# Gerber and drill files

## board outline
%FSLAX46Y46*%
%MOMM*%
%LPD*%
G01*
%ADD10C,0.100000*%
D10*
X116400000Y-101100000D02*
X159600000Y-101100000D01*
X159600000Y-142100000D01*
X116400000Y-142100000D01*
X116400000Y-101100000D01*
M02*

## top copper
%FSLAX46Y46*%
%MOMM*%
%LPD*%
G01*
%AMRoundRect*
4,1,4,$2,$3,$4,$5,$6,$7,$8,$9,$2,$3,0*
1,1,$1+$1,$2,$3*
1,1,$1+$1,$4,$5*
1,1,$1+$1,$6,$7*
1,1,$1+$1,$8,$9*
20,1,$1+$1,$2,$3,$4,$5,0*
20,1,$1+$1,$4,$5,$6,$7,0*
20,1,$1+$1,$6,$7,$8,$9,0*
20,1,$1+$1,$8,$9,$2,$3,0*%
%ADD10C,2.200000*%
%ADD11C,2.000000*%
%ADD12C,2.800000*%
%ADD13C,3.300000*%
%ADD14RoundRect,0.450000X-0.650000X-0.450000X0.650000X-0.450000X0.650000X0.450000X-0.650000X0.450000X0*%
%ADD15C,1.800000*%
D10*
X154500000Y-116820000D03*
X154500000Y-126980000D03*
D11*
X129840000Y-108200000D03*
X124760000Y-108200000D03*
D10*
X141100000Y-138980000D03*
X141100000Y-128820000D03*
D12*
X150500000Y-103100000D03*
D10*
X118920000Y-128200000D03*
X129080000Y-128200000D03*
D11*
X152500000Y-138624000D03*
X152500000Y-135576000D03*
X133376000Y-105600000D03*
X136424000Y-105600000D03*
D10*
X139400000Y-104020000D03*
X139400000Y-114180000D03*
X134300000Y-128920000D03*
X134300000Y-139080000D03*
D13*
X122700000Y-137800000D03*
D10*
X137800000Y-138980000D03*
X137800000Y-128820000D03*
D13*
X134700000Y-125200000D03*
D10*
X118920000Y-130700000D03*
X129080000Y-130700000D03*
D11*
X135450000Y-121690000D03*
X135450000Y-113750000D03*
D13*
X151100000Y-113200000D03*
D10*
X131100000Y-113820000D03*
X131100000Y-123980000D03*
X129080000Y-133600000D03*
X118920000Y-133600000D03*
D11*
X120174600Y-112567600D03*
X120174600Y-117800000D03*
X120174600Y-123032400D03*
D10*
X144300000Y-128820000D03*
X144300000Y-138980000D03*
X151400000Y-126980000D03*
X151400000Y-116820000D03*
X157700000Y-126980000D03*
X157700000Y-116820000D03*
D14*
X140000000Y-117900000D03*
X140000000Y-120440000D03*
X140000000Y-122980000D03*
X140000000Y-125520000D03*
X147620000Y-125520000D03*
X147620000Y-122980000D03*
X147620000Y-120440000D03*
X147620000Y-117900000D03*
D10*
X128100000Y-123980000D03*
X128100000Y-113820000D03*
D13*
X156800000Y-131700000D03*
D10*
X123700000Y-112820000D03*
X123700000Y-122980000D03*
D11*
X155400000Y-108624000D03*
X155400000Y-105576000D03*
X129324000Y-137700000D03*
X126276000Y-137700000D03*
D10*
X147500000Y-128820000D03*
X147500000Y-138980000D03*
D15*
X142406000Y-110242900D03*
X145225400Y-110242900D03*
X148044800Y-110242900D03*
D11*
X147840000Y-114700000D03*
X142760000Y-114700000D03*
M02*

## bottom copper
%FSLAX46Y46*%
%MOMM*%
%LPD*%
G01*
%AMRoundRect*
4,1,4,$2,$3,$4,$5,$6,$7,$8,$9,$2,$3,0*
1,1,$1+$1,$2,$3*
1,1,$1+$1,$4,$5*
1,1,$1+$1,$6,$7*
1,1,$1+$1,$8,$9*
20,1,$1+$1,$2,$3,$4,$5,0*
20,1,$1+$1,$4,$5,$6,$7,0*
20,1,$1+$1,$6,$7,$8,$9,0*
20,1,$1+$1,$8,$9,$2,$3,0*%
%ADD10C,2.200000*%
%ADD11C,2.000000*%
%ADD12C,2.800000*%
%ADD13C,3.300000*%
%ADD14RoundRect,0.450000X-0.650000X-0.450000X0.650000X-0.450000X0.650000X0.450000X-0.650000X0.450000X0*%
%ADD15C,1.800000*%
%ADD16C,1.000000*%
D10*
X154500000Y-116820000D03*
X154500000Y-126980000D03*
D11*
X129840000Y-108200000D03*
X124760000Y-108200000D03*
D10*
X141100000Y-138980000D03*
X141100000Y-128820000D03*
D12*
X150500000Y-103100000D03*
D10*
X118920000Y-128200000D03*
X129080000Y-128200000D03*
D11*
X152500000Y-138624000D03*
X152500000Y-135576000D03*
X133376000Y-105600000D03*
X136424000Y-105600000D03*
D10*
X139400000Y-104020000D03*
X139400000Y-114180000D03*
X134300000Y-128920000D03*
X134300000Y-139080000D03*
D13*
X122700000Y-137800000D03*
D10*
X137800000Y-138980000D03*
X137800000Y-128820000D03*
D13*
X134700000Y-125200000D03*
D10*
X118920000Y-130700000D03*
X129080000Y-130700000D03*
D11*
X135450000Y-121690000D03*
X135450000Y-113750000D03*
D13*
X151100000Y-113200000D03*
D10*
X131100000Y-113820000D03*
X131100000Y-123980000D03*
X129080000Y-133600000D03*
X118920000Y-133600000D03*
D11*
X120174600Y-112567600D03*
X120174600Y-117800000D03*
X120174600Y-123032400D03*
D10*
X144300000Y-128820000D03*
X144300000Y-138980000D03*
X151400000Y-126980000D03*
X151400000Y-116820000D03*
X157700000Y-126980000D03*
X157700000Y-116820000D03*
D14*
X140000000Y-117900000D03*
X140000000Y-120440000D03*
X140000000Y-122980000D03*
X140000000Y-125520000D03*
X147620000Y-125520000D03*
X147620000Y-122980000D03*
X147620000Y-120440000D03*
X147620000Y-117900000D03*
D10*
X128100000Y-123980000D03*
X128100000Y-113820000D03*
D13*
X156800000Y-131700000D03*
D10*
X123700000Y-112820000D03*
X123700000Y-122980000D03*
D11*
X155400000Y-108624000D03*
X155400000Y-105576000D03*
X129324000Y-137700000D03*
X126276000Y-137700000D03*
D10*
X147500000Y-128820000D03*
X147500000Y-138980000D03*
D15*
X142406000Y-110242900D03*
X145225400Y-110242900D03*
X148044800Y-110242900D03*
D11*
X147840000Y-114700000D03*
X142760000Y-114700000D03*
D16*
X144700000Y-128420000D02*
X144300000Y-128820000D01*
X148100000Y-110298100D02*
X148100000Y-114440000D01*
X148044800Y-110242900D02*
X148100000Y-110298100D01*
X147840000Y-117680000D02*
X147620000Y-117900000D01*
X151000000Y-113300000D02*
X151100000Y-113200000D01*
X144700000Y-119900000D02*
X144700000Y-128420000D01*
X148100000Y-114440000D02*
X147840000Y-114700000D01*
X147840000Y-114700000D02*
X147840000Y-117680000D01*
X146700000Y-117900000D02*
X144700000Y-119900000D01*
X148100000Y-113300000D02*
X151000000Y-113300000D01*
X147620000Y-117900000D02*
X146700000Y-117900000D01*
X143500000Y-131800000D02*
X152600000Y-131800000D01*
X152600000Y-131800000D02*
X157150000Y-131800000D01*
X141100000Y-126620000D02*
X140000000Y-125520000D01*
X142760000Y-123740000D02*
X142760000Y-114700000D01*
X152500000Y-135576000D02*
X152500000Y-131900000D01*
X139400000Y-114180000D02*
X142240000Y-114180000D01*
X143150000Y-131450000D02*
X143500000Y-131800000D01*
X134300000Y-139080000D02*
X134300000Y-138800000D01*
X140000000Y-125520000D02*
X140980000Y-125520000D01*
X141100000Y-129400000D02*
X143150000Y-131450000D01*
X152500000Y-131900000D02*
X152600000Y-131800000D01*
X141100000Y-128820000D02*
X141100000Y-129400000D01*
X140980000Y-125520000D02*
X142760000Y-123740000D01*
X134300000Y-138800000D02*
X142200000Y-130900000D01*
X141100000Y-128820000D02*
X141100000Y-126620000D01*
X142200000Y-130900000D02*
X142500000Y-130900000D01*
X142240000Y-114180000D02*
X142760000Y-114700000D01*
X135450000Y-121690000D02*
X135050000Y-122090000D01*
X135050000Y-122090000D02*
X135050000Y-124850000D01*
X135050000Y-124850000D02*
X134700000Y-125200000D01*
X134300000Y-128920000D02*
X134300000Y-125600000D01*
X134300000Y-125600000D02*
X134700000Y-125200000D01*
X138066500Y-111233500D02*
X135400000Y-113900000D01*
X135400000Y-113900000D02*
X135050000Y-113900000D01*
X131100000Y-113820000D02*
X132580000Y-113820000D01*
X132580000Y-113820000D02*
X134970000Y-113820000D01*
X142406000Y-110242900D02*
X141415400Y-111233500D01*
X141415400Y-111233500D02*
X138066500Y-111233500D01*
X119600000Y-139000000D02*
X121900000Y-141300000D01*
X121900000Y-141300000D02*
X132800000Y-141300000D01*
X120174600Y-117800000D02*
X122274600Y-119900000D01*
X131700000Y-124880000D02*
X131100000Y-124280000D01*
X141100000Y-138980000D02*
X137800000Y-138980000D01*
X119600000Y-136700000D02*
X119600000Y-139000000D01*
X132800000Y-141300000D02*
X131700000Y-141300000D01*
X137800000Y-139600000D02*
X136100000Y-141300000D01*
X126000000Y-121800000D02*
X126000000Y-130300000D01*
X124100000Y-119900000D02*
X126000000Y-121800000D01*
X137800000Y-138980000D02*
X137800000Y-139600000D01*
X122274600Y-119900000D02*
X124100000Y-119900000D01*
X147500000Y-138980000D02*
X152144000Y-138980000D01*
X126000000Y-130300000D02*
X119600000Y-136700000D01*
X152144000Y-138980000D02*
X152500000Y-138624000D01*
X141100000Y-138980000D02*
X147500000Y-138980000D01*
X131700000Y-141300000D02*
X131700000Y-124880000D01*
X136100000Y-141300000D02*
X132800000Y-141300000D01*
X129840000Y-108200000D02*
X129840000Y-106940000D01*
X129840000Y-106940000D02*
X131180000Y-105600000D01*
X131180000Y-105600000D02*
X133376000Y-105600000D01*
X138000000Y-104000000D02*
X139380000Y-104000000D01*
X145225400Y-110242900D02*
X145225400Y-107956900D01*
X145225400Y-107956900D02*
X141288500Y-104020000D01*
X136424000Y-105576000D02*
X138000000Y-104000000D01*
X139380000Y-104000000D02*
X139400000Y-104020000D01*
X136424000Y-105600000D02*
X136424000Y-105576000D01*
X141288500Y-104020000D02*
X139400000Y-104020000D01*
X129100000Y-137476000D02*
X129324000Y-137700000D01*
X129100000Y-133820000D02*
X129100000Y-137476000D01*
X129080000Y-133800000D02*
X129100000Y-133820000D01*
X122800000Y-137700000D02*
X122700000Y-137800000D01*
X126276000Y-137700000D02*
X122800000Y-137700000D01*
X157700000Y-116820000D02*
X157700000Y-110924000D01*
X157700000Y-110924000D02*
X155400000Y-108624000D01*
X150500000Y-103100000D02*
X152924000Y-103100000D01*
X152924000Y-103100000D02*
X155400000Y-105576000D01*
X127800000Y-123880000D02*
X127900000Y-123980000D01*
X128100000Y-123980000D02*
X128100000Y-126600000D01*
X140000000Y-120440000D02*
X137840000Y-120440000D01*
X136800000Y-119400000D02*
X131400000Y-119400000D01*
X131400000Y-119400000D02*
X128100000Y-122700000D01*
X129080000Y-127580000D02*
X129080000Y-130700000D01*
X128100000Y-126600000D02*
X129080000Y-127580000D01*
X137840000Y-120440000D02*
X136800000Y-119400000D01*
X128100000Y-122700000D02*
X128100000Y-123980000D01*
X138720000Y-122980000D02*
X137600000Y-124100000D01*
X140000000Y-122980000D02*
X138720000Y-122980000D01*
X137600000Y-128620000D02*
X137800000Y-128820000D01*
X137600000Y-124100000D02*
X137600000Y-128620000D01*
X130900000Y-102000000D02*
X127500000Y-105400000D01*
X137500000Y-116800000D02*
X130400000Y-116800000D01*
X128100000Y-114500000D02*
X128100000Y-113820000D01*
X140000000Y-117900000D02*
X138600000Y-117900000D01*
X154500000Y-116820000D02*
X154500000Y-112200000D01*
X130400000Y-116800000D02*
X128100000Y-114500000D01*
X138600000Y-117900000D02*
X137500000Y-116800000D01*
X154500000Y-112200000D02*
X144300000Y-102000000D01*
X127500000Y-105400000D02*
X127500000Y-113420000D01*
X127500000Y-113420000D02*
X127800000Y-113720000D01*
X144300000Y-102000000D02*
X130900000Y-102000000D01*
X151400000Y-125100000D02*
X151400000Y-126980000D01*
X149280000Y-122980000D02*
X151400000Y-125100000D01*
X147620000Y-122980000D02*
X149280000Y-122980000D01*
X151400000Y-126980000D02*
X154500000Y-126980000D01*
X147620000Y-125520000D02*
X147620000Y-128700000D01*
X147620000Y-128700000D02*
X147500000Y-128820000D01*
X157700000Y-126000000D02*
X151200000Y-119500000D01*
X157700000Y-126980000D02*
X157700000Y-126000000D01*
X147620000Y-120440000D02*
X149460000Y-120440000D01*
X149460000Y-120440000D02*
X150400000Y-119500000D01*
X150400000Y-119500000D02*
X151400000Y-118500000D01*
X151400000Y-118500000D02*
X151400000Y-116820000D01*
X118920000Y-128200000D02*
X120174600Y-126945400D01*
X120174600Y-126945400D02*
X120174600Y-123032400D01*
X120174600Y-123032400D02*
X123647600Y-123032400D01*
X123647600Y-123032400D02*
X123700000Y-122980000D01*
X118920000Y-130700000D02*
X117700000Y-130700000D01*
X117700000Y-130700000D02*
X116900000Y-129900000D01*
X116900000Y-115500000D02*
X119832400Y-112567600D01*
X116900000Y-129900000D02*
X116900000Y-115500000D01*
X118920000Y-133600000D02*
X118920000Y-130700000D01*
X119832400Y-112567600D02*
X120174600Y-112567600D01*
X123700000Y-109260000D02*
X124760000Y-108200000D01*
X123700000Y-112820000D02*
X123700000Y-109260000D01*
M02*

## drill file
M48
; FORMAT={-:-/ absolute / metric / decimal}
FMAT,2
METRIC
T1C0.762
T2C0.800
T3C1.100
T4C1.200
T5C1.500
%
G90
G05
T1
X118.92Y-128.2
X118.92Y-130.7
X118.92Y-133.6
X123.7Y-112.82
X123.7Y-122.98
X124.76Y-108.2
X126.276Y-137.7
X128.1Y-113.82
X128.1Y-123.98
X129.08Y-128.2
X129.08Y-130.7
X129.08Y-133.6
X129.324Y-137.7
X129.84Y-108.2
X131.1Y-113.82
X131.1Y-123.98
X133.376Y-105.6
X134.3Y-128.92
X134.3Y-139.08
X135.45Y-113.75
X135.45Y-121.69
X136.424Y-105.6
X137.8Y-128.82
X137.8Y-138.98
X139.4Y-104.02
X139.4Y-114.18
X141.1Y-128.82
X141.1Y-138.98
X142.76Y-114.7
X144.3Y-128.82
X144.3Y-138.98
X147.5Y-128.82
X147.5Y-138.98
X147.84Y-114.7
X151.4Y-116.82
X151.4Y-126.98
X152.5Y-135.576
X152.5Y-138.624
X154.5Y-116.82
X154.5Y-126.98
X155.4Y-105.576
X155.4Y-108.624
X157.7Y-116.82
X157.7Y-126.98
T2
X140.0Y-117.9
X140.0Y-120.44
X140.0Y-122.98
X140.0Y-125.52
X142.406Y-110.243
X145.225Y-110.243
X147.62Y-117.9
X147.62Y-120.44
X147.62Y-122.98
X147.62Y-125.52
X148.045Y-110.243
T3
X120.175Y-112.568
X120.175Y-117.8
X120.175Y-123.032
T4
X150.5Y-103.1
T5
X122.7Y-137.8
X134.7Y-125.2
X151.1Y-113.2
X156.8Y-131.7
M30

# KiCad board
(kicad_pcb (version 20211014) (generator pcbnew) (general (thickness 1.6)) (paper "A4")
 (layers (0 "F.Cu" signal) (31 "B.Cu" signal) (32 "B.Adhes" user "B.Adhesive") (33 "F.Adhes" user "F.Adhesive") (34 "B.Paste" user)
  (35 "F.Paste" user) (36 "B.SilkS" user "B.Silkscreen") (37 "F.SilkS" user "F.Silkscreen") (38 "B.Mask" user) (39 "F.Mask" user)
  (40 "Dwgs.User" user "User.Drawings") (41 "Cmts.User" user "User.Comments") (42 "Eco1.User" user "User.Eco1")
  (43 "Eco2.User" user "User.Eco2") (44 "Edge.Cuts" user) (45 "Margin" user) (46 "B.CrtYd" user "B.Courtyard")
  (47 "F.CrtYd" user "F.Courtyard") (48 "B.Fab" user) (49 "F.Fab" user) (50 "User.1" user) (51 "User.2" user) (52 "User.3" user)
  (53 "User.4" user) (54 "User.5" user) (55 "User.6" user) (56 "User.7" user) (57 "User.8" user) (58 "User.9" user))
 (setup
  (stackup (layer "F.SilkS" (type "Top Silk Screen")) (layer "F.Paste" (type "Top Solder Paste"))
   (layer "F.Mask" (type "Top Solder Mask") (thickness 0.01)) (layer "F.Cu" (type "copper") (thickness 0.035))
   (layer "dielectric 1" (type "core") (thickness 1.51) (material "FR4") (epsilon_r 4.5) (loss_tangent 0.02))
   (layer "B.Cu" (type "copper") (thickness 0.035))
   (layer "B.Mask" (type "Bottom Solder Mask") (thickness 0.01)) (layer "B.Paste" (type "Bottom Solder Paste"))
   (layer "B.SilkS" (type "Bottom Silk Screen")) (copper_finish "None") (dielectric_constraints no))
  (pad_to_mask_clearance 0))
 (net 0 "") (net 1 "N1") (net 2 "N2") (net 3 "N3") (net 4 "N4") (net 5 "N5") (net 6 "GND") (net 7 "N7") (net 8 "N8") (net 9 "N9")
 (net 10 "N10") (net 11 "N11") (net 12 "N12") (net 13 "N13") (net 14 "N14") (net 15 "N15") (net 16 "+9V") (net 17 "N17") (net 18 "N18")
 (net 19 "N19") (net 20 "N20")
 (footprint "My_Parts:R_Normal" (layer "F.Cu") (at 154.5 121.9 -90)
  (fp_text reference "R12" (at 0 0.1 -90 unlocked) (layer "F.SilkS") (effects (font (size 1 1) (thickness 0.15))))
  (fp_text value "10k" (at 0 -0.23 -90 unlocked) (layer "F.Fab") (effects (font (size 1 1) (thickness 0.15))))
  (pad "1" thru_hole circle (at -5.08 0 270) (size 2.2 2.2) (drill 0.762) (layers *.Cu *.Mask) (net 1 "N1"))
  (pad "2" thru_hole circle (at 5.08 0 270) (size 2.2 2.2) (drill 0.762) (layers *.Cu *.Mask) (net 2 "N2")))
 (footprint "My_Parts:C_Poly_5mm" (layer "F.Cu") (at 127.3 108.2 180)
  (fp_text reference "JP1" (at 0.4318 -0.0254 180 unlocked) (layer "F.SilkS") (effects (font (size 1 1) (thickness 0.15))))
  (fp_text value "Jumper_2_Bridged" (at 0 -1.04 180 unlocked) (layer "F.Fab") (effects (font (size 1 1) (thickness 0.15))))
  (pad "1" thru_hole circle (at -2.54 0 180) (size 2 2) (drill 0.762) (layers *.Cu *.Mask) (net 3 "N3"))
  (pad "2" thru_hole circle (at 2.54 0 180) (size 2 2) (drill 0.762) (layers *.Cu *.Mask) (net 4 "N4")))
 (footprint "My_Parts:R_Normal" (layer "F.Cu") (at 141.1 133.9 90)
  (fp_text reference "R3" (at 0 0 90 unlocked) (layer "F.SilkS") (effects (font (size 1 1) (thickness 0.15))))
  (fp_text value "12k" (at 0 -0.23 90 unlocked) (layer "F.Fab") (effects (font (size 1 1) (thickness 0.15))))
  (pad "1" thru_hole circle (at -5.08 0 90) (size 2.2 2.2) (drill 0.762) (layers *.Cu *.Mask) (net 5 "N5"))
  (pad "2" thru_hole circle (at 5.08 0 90) (size 2.2 2.2) (drill 0.762) (layers *.Cu *.Mask) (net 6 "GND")))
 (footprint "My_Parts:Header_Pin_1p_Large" (layer "F.Cu") (at 150.5 103.1)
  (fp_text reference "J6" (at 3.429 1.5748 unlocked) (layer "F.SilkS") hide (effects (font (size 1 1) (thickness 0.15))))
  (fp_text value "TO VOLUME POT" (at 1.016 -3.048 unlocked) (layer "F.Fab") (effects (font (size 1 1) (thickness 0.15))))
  (pad "1" thru_hole circle (at 0 0) (size 2.8 2.8) (drill 1.2) (layers *.Cu *.Mask) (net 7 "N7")))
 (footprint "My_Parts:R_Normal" (layer "F.Cu") (at 124 128.2)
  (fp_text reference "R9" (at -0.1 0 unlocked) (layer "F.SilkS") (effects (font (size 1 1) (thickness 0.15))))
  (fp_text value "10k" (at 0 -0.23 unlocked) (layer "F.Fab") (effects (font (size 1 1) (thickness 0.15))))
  (pad "1" thru_hole circle (at -5.08 0) (size 2.2 2.2) (drill 0.762) (layers *.Cu *.Mask) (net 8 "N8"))
  (pad "2" thru_hole circle (at 5.08 0) (size 2.2 2.2) (drill 0.762) (layers *.Cu *.Mask) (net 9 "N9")))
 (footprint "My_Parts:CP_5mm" (layer "F.Cu") (at 152.5 137.1 90)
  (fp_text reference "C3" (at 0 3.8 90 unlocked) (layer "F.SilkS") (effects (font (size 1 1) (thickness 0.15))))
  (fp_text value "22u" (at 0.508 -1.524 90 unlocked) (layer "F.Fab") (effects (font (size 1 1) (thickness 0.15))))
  (pad "1" thru_hole circle (at -1.524 0 90) (size 2 2) (drill 0.762) (layers *.Cu *.Mask) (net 5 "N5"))
  (pad "2" thru_hole circle (at 1.524 0 90) (size 2 2) (drill 0.762) (layers *.Cu *.Mask) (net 6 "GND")))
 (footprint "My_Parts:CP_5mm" (layer "F.Cu") (at 134.9 105.6)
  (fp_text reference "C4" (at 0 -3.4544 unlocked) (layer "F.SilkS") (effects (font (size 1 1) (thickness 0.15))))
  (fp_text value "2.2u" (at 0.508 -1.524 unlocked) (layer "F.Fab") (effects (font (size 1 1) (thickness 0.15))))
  (pad "1" thru_hole circle (at -1.524 0) (size 2 2) (drill 0.762) (layers *.Cu *.Mask) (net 3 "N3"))
  (pad "2" thru_hole circle (at 1.524 0) (size 2 2) (drill 0.762) (layers *.Cu *.Mask) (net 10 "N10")))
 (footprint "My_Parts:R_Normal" (layer "F.Cu") (at 139.4 109.1 -90)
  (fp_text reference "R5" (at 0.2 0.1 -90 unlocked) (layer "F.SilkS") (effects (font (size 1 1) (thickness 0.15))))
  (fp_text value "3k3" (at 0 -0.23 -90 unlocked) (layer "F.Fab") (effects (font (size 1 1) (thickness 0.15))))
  (pad "1" thru_hole circle (at -5.08 0 270) (size 2.2 2.2) (drill 0.762) (layers *.Cu *.Mask) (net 10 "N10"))
  (pad "2" thru_hole circle (at 5.08 0 270) (size 2.2 2.2) (drill 0.762) (layers *.Cu *.Mask) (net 6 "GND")))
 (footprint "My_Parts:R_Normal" (layer "F.Cu") (at 134.3 134 -90)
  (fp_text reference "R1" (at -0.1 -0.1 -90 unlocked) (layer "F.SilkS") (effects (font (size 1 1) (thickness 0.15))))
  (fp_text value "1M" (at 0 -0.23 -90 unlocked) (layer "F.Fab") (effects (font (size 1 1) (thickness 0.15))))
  (pad "1" thru_hole circle (at -5.08 0 270) (size 2.2 2.2) (drill 0.762) (layers *.Cu *.Mask) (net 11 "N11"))
  (pad "2" thru_hole circle (at 5.08 0 270) (size 2.2 2.2) (drill 0.762) (layers *.Cu *.Mask) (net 6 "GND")))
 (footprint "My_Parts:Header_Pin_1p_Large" (layer "F.Cu") (at 122.7 137.8)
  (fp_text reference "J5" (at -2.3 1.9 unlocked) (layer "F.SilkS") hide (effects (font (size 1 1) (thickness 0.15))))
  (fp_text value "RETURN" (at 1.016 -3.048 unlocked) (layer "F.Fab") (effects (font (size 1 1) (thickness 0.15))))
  (pad "1" thru_hole circle (at 0 0) (size 3.3 3.3) (drill 1.5) (layers *.Cu *.Mask) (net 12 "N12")))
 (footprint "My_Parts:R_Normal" (layer "F.Cu") (at 137.8 133.9 90)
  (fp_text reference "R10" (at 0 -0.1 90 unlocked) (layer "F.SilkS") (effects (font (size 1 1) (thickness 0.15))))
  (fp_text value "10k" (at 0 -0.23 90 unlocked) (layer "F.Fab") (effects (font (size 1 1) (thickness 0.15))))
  (pad "1" thru_hole circle (at -5.08 0 90) (size 2.2 2.2) (drill 0.762) (layers *.Cu *.Mask) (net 5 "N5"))
  (pad "2" thru_hole circle (at 5.08 0 90) (size 2.2 2.2) (drill 0.762) (layers *.Cu *.Mask) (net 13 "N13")))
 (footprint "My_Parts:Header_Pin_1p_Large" (layer "F.Cu") (at 134.7 125.2)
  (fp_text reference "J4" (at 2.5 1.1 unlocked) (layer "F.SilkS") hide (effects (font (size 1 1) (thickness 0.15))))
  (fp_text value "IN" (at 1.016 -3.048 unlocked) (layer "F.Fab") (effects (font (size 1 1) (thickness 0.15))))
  (pad "1" thru_hole circle (at 0 0) (size 3.3 3.3) (drill 1.5) (layers *.Cu *.Mask) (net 11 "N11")))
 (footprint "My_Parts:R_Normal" (layer "F.Cu") (at 124 130.7)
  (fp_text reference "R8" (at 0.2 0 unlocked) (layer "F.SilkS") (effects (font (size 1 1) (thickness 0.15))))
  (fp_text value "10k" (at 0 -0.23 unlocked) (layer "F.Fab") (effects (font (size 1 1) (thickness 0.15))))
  (pad "1" thru_hole circle (at -5.08 0) (size 2.2 2.2) (drill 0.762) (layers *.Cu *.Mask) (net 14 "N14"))
  (pad "2" thru_hole circle (at 5.08 0) (size 2.2 2.2) (drill 0.762) (layers *.Cu *.Mask) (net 9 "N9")))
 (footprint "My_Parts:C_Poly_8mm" (layer "F.Cu") (at 135.45 119.15 90)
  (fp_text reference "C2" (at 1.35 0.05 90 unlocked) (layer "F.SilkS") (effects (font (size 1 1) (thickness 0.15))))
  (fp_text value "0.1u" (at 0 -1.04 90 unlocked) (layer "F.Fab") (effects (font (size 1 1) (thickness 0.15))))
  (pad "1" thru_hole circle (at -2.54 0 90) (size 2 2) (drill 0.762) (layers *.Cu *.Mask) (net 11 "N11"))
  (pad "2" thru_hole circle (at 5.4 0 90) (size 2 2) (drill 0.762) (layers *.Cu *.Mask) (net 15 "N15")))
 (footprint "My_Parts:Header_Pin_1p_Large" (layer "F.Cu") (at 151.1 113.2)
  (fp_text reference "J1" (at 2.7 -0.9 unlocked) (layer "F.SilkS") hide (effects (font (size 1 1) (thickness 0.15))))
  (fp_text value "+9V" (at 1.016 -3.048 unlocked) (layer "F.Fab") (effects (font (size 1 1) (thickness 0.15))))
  (pad "1" thru_hole circle (at 0 0) (size 3.3 3.3) (drill 1.5) (layers *.Cu *.Mask) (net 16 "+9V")))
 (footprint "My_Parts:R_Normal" (layer "F.Cu") (at 131.1 118.9 -90)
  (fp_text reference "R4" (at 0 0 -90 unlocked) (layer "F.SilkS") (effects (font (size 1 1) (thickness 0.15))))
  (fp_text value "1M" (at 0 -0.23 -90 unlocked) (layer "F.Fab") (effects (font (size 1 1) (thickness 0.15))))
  (pad "1" thru_hole circle (at -5.08 0 270) (size 2.2 2.2) (drill 0.762) (layers *.Cu *.Mask) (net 15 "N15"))
  (pad "2" thru_hole circle (at 5.08 0 270) (size 2.2 2.2) (drill 0.762) (layers *.Cu *.Mask) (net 5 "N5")))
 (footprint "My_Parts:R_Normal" (layer "F.Cu") (at 124 133.6 180)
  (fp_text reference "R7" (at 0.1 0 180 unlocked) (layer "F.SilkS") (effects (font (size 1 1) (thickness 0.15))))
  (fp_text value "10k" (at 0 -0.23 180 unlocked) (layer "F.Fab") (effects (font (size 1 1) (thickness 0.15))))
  (pad "1" thru_hole circle (at -5.08 0 180) (size 2.2 2.2) (drill 0.762) (layers *.Cu *.Mask) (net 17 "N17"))
  (pad "2" thru_hole circle (at 5.08 0 180) (size 2.2 2.2) (drill 0.762) (layers *.Cu *.Mask) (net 14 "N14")))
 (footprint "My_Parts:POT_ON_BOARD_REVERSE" (layer "F.Cu") (at 120.2 117.8 90)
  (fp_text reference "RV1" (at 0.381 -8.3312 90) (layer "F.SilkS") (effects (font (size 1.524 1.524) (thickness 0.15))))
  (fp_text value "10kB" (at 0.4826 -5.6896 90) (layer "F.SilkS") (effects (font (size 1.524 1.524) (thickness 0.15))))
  (pad "1" thru_hole circle (at 5.2324 -0.0254 90) (size 2 2) (drill 1.09982) (layers *.Cu "F.Paste" "F.Mask") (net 14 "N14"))
  (pad "2" thru_hole circle (at 0 -0.0254 90) (size 2 2) (drill 1.09982) (layers *.Cu "F.Paste" "F.Mask") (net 5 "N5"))
  (pad "3" thru_hole circle (at -5.2324 -0.0254 90) (size 2 2) (drill 1.09982) (layers *.Cu "F.Paste" "F.Mask") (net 8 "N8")))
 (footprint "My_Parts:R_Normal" (layer "F.Cu") (at 144.3 133.9 -90)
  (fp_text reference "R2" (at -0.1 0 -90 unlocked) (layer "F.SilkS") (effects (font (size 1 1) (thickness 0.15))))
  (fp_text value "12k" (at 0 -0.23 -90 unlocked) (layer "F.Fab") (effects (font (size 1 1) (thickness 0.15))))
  (pad "1" thru_hole circle (at -5.08 0 270) (size 2.2 2.2) (drill 0.762) (layers *.Cu *.Mask) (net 16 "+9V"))
  (pad "2" thru_hole circle (at 5.08 0 270) (size 2.2 2.2) (drill 0.762) (layers *.Cu *.Mask) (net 5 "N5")))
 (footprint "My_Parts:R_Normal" (layer "F.Cu") (at 151.4 121.9 90)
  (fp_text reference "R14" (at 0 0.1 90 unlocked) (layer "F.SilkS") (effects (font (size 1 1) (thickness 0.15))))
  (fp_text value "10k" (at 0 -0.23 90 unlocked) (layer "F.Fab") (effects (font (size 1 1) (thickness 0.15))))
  (pad "1" thru_hole circle (at -5.08 0 90) (size 2.2 2.2) (drill 0.762) (layers *.Cu *.Mask) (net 2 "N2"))
  (pad "2" thru_hole circle (at 5.08 0 90) (size 2.2 2.2) (drill 0.762) (layers *.Cu *.Mask) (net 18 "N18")))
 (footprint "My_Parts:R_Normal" (layer "F.Cu") (at 157.7 121.9 90)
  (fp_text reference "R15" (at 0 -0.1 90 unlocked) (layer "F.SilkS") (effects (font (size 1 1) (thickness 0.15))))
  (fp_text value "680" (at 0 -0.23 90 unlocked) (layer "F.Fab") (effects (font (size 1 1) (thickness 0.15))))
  (pad "1" thru_hole circle (at -5.08 0 90) (size 2.2 2.2) (drill 0.762) (layers *.Cu *.Mask) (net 18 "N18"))
  (pad "2" thru_hole circle (at 5.08 0 90) (size 2.2 2.2) (drill 0.762) (layers *.Cu *.Mask) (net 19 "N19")))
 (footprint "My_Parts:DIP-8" (layer "F.Cu") (at 141.27 118.4)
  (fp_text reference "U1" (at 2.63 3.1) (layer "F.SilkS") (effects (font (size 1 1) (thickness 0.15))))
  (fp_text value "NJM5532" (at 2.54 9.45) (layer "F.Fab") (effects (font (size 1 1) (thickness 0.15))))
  (pad "1" thru_hole roundrect (at -1.27 -0.5) (size 2.2 1.8) (drill 0.8) (layers *.Cu *.Mask) (roundrect_rratio 0.25) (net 1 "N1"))
  (pad "2" thru_hole roundrect (at -1.27 2.04) (size 2.2 1.8) (drill 0.8) (layers *.Cu *.Mask) (roundrect_rratio 0.25) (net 9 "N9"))
  (pad "3" thru_hole roundrect (at -1.27 4.58) (size 2.2 1.8) (drill 0.8) (layers *.Cu *.Mask) (roundrect_rratio 0.25) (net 13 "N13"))
  (pad "4" thru_hole roundrect (at -1.27 7.12) (size 2.2 1.8) (drill 0.8) (layers *.Cu *.Mask) (roundrect_rratio 0.25) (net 6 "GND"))
  (pad "5" thru_hole roundrect (at 6.35 7.12) (size 2.2 1.8) (drill 0.8) (layers *.Cu *.Mask) (roundrect_rratio 0.25) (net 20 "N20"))
  (pad "6" thru_hole roundrect (at 6.35 4.58) (size 2.2 1.8) (drill 0.8) (layers *.Cu *.Mask) (roundrect_rratio 0.25) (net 2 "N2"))
  (pad "7" thru_hole roundrect (at 6.35 2.04) (size 2.2 1.8) (drill 0.8) (layers *.Cu *.Mask) (roundrect_rratio 0.25) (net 18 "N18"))
  (pad "8" thru_hole roundrect (at 6.35 -0.5) (size 2.2 1.8) (drill 0.8) (layers *.Cu *.Mask) (roundrect_rratio 0.25) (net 16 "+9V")))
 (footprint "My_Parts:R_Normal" (layer "F.Cu") (at 128.1 118.9 90)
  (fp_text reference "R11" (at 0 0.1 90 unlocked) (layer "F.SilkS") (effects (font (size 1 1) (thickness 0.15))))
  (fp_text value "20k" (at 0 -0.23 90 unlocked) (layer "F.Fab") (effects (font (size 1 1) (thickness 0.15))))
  (pad "1" thru_hole circle (at -5.08 0 90) (size 2.2 2.2) (drill 0.762) (layers *.Cu *.Mask) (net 9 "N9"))
  (pad "2" thru_hole circle (at 5.08 0 90) (size 2.2 2.2) (drill 0.762) (layers *.Cu *.Mask) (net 1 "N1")))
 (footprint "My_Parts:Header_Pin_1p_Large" (layer "F.Cu") (at 156.8 131.7)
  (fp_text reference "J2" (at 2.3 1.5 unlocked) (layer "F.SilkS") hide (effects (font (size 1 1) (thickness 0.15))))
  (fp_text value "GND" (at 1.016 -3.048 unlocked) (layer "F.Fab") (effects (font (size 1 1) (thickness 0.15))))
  (pad "1" thru_hole circle (at 0 0) (size 3.3 3.3) (drill 1.5) (layers *.Cu *.Mask) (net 6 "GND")))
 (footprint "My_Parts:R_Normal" (layer "F.Cu") (at 123.7 117.9 -90)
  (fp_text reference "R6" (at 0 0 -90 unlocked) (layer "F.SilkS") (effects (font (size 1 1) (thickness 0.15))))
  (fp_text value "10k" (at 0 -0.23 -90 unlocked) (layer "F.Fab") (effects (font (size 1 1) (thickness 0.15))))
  (pad "1" thru_hole circle (at -5.08 0 270) (size 2.2 2.2) (drill 0.762) (layers *.Cu *.Mask) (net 4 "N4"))
  (pad "2" thru_hole circle (at 5.08 0 270) (size 2.2 2.2) (drill 0.762) (layers *.Cu *.Mask) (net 8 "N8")))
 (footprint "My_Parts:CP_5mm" (layer "F.Cu") (at 155.4 107.1 90)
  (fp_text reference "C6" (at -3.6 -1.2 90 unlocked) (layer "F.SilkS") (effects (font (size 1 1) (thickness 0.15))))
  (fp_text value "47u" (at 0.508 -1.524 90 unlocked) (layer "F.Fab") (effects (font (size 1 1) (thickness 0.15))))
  (pad "1" thru_hole circle (at -1.524 0 90) (size 2 2) (drill 0.762) (layers *.Cu *.Mask) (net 19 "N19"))
  (pad "2" thru_hole circle (at 1.524 0 90) (size 2 2) (drill 0.762) (layers *.Cu *.Mask) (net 7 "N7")))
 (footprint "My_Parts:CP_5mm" (layer "F.Cu") (at 127.8 137.7 180)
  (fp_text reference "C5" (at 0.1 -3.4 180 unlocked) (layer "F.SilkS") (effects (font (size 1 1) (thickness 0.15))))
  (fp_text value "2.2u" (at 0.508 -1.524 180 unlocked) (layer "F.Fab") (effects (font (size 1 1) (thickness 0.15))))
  (pad "1" thru_hole circle (at -1.524 0 180) (size 2 2) (drill 0.762) (layers *.Cu *.Mask) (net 17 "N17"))
  (pad "2" thru_hole circle (at 1.524 0 180) (size 2 2) (drill 0.762) (layers *.Cu *.Mask) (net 12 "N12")))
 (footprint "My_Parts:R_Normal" (layer "F.Cu") (at 147.5 133.9 -90)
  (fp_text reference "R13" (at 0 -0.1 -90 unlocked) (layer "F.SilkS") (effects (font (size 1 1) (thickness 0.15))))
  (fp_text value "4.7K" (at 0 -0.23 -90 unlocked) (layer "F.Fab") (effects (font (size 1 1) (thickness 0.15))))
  (pad "1" thru_hole circle (at -5.08 0 270) (size 2.2 2.2) (drill 0.762) (layers *.Cu *.Mask) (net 20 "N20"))
  (pad "2" thru_hole circle (at 5.08 0 270) (size 2.2 2.2) (drill 0.762) (layers *.Cu *.Mask) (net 5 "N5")))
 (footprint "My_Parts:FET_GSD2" (layer "F.Cu") (at 142.66 110.2175)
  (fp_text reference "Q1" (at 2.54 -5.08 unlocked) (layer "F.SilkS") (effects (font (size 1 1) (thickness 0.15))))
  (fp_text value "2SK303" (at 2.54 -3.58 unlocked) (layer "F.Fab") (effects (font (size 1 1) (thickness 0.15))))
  (pad "1" thru_hole circle (at -0.254 0.0254) (size 1.8 1.8) (drill 0.8) (layers *.Cu *.Mask) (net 15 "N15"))
  (pad "2" thru_hole circle (at 2.5654 0.0254) (size 1.8 1.8) (drill 0.8) (layers *.Cu *.Mask) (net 10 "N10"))
  (pad "3" thru_hole circle (at 5.3848 0.0254) (size 1.8 1.8) (drill 0.8) (layers *.Cu *.Mask) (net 16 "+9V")))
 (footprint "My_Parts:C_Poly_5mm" (layer "F.Cu") (at 145.3 114.7 180)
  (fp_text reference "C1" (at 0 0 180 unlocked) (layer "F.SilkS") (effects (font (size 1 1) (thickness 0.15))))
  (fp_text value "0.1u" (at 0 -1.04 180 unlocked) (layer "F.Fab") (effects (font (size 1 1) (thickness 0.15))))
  (pad "1" thru_hole circle (at -2.54 0 180) (size 2 2) (drill 0.762) (layers *.Cu *.Mask) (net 16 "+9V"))
  (pad "2" thru_hole circle (at 2.54 0 180) (size 2 2) (drill 0.762) (layers *.Cu *.Mask) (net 6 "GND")))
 (gr_rect (start 116.4 101.1) (end 159.6 142.1) (layer "Edge.Cuts") (width 0.1) (fill none))
 (segment (start 144.7 128.42) (end 144.3 128.82) (width 1) (layer "B.Cu") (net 16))
 (segment (start 148.1 110.2981) (end 148.1 114.44) (width 1) (layer "B.Cu") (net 16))
 (segment (start 148.0448 110.2429) (end 148.1 110.2981) (width 1) (layer "B.Cu") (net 16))
 (segment (start 147.84 117.68) (end 147.62 117.9) (width 1) (layer "B.Cu") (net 16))
 (segment (start 151 113.3) (end 151.1 113.2) (width 1) (layer "B.Cu") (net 16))
 (segment (start 144.7 119.9) (end 144.7 128.42) (width 1) (layer "B.Cu") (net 16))
 (segment (start 148.1 114.44) (end 147.84 114.7) (width 1) (layer "B.Cu") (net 16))
 (segment (start 147.84 114.7) (end 147.84 117.68) (width 1) (layer "B.Cu") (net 16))
 (segment (start 146.7 117.9) (end 144.7 119.9) (width 1) (layer "B.Cu") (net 16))
 (segment (start 148.1 113.3) (end 151 113.3) (width 1) (layer "B.Cu") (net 16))
 (segment (start 147.62 117.9) (end 146.7 117.9) (width 1) (layer "B.Cu") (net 16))
 (segment (start 143.5 131.8) (end 152.6 131.8) (width 1) (layer "B.Cu") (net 6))
 (segment (start 152.6 131.8) (end 157.15 131.8) (width 1) (layer "B.Cu") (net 6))
 (segment (start 141.1 126.62) (end 140 125.52) (width 1) (layer "B.Cu") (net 6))
 (segment (start 142.76 123.74) (end 142.76 114.7) (width 1) (layer "B.Cu") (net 6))
 (segment (start 152.5 135.576) (end 152.5 131.9) (width 1) (layer "B.Cu") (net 6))
 (segment (start 139.4 114.18) (end 142.24 114.18) (width 1) (layer "B.Cu") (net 6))
 (segment (start 143.15 131.45) (end 143.5 131.8) (width 1) (layer "B.Cu") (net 6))
 (segment (start 134.3 139.08) (end 134.3 138.8) (width 1) (layer "B.Cu") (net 6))
 (segment (start 140 125.52) (end 140.98 125.52) (width 1) (layer "B.Cu") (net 6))
 (segment (start 141.1 129.4) (end 143.15 131.45) (width 1) (layer "B.Cu") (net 6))
 (segment (start 152.5 131.9) (end 152.6 131.8) (width 1) (layer "B.Cu") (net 6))
 (segment (start 141.1 128.82) (end 141.1 129.4) (width 1) (layer "B.Cu") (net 6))
 (segment (start 140.98 125.52) (end 142.76 123.74) (width 1) (layer "B.Cu") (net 6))
 (segment (start 134.3 138.8) (end 142.2 130.9) (width 1) (layer "B.Cu") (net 6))
 (segment (start 141.1 128.82) (end 141.1 126.62) (width 1) (layer "B.Cu") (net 6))
 (segment (start 142.2 130.9) (end 142.5 130.9) (width 1) (layer "B.Cu") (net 6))
 (segment (start 142.24 114.18) (end 142.76 114.7) (width 1) (layer "B.Cu") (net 6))
 (segment (start 135.45 121.69) (end 135.05 122.09) (width 1) (layer "B.Cu") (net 11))
 (segment (start 135.05 122.09) (end 135.05 124.85) (width 1) (layer "B.Cu") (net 11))
 (segment (start 135.05 124.85) (end 134.7 125.2) (width 1) (layer "B.Cu") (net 11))
 (segment (start 134.3 128.92) (end 134.3 125.6) (width 1) (layer "B.Cu") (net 11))
 (segment (start 134.3 125.6) (end 134.7 125.2) (width 1) (layer "B.Cu") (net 11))
 (segment (start 138.0665 111.2335) (end 135.4 113.9) (width 1) (layer "B.Cu") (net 15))
 (segment (start 135.4 113.9) (end 135.05 113.9) (width 1) (layer "B.Cu") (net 15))
 (segment (start 131.1 113.82) (end 132.58 113.82) (width 1) (layer "B.Cu") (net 15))
 (segment (start 132.58 113.82) (end 134.97 113.82) (width 1) (layer "B.Cu") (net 15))
 (segment (start 142.406 110.2429) (end 141.4154 111.2335) (width 1) (layer "B.Cu") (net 15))
 (segment (start 141.4154 111.2335) (end 138.0665 111.2335) (width 1) (layer "B.Cu") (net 15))
 (segment (start 119.6 139) (end 121.9 141.3) (width 1) (layer "B.Cu") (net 5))
 (segment (start 121.9 141.3) (end 132.8 141.3) (width 1) (layer "B.Cu") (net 5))
 (segment (start 120.1746 117.8) (end 122.2746 119.9) (width 1) (layer "B.Cu") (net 5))
 (segment (start 131.7 124.88) (end 131.1 124.28) (width 1) (layer "B.Cu") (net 5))
 (segment (start 141.1 138.98) (end 137.8 138.98) (width 1) (layer "B.Cu") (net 5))
 (segment (start 119.6 136.7) (end 119.6 139) (width 1) (layer "B.Cu") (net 5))
 (segment (start 132.8 141.3) (end 131.7 141.3) (width 1) (layer "B.Cu") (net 5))
 (segment (start 137.8 139.6) (end 136.1 141.3) (width 1) (layer "B.Cu") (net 5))
 (segment (start 126 121.8) (end 126 130.3) (width 1) (layer "B.Cu") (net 5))
 (segment (start 124.1 119.9) (end 126 121.8) (width 1) (layer "B.Cu") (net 5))
 (segment (start 137.8 138.98) (end 137.8 139.6) (width 1) (layer "B.Cu") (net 5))
 (segment (start 122.2746 119.9) (end 124.1 119.9) (width 1) (layer "B.Cu") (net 5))
 (segment (start 147.5 138.98) (end 152.144 138.98) (width 1) (layer "B.Cu") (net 5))
 (segment (start 126 130.3) (end 119.6 136.7) (width 1) (layer "B.Cu") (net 5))
 (segment (start 152.144 138.98) (end 152.5 138.624) (width 1) (layer "B.Cu") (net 5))
 (segment (start 141.1 138.98) (end 147.5 138.98) (width 1) (layer "B.Cu") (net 5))
 (segment (start 131.7 141.3) (end 131.7 124.88) (width 1) (layer "B.Cu") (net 5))
 (segment (start 136.1 141.3) (end 132.8 141.3) (width 1) (layer "B.Cu") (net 5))
 (segment (start 129.84 108.2) (end 129.84 106.94) (width 1) (layer "B.Cu") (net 3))
 (segment (start 129.84 106.94) (end 131.18 105.6) (width 1) (layer "B.Cu") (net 3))
 (segment (start 131.18 105.6) (end 133.376 105.6) (width 1) (layer "B.Cu") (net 3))
 (segment (start 138 104) (end 139.38 104) (width 1) (layer "B.Cu") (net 10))
 (segment (start 145.2254 110.2429) (end 145.2254 107.9569) (width 1) (layer "B.Cu") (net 10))
 (segment (start 145.2254 107.9569) (end 141.2885 104.02) (width 1) (layer "B.Cu") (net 10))
 (segment (start 136.424 105.576) (end 138 104) (width 1) (layer "B.Cu") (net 10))
 (segment (start 139.38 104) (end 139.4 104.02) (width 1) (layer "B.Cu") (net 10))
 (segment (start 136.424 105.6) (end 136.424 105.576) (width 1) (layer "B.Cu") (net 10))
 (segment (start 141.2885 104.02) (end 139.4 104.02) (width 1) (layer "B.Cu") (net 10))
 (segment (start 129.1 137.476) (end 129.324 137.7) (width 1) (layer "B.Cu") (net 17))
 (segment (start 129.1 133.82) (end 129.1 137.476) (width 1) (layer "B.Cu") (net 17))
 (segment (start 129.08 133.8) (end 129.1 133.82) (width 1) (layer "B.Cu") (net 17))
 (segment (start 122.8 137.7) (end 122.7 137.8) (width 1) (layer "B.Cu") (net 12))
 (segment (start 126.276 137.7) (end 122.8 137.7) (width 1) (layer "B.Cu") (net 12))
 (segment (start 157.7 116.82) (end 157.7 110.924) (width 1) (layer "B.Cu") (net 19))
 (segment (start 157.7 110.924) (end 155.4 108.624) (width 1) (layer "B.Cu") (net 19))
 (segment (start 150.5 103.1) (end 152.924 103.1) (width 1) (layer "B.Cu") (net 7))
 (segment (start 152.924 103.1) (end 155.4 105.576) (width 1) (layer "B.Cu") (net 7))
 (segment (start 127.8 123.88) (end 127.9 123.98) (width 1) (layer "B.Cu") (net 9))
 (segment (start 128.1 123.98) (end 128.1 126.6) (width 1) (layer "B.Cu") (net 9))
 (segment (start 140 120.44) (end 137.84 120.44) (width 1) (layer "B.Cu") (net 9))
 (segment (start 136.8 119.4) (end 131.4 119.4) (width 1) (layer "B.Cu") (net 9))
 (segment (start 131.4 119.4) (end 128.1 122.7) (width 1) (layer "B.Cu") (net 9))
 (segment (start 129.08 127.58) (end 129.08 130.7) (width 1) (layer "B.Cu") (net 9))
 (segment (start 128.1 126.6) (end 129.08 127.58) (width 1) (layer "B.Cu") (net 9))
 (segment (start 137.84 120.44) (end 136.8 119.4) (width 1) (layer "B.Cu") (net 9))
 (segment (start 128.1 122.7) (end 128.1 123.98) (width 1) (layer "B.Cu") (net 9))
 (segment (start 138.72 122.98) (end 137.6 124.1) (width 1) (layer "B.Cu") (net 13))
 (segment (start 140 122.98) (end 138.72 122.98) (width 1) (layer "B.Cu") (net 13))
 (segment (start 137.6 128.62) (end 137.8 128.82) (width 1) (layer "B.Cu") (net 13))
 (segment (start 137.6 124.1) (end 137.6 128.62) (width 1) (layer "B.Cu") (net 13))
 (segment (start 130.9 102) (end 127.5 105.4) (width 1) (layer "B.Cu") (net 1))
 (segment (start 137.5 116.8) (end 130.4 116.8) (width 1) (layer "B.Cu") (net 1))
 (segment (start 128.1 114.5) (end 128.1 113.82) (width 1) (layer "B.Cu") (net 1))
 (segment (start 140 117.9) (end 138.6 117.9) (width 1) (layer "B.Cu") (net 1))
 (segment (start 154.5 116.82) (end 154.5 112.2) (width 1) (layer "B.Cu") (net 1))
 (segment (start 130.4 116.8) (end 128.1 114.5) (width 1) (layer "B.Cu") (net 1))
 (segment (start 138.6 117.9) (end 137.5 116.8) (width 1) (layer "B.Cu") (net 1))
 (segment (start 154.5 112.2) (end 144.3 102) (width 1) (layer "B.Cu") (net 1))
 (segment (start 127.5 105.4) (end 127.5 113.42) (width 1) (layer "B.Cu") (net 1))
 (segment (start 127.5 113.42) (end 127.8 113.72) (width 1) (layer "B.Cu") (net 1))
 (segment (start 144.3 102) (end 130.9 102) (width 1) (layer "B.Cu") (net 1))
 (segment (start 151.4 125.1) (end 151.4 126.98) (width 1) (layer "B.Cu") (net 2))
 (segment (start 149.28 122.98) (end 151.4 125.1) (width 1) (layer "B.Cu") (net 2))
 (segment (start 147.62 122.98) (end 149.28 122.98) (width 1) (layer "B.Cu") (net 2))
 (segment (start 151.4 126.98) (end 154.5 126.98) (width 1) (layer "B.Cu") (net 2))
 (segment (start 147.62 125.52) (end 147.62 128.7) (width 1) (layer "B.Cu") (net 20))
 (segment (start 147.62 128.7) (end 147.5 128.82) (width 1) (layer "B.Cu") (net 20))
 (segment (start 157.7 126) (end 151.2 119.5) (width 1) (layer "B.Cu") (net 18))
 (segment (start 157.7 126.98) (end 157.7 126) (width 1) (layer "B.Cu") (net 18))
 (segment (start 147.62 120.44) (end 149.46 120.44) (width 1) (layer "B.Cu") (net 18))
 (segment (start 149.46 120.44) (end 150.4 119.5) (width 1) (layer "B.Cu") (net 18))
 (segment (start 150.4 119.5) (end 151.4 118.5) (width 1) (layer "B.Cu") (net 18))
 (segment (start 151.4 118.5) (end 151.4 116.82) (width 1) (layer "B.Cu") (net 18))
 (segment (start 118.92 128.2) (end 120.1746 126.9454) (width 1) (layer "B.Cu") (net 8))
 (segment (start 120.1746 126.9454) (end 120.1746 123.0324) (width 1) (layer "B.Cu") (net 8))
 (segment (start 120.1746 123.0324) (end 123.6476 123.0324) (width 1) (layer "B.Cu") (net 8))
 (segment (start 123.6476 123.0324) (end 123.7 122.98) (width 1) (layer "B.Cu") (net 8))
 (segment (start 118.92 130.7) (end 117.7 130.7) (width 1) (layer "B.Cu") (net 14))
 (segment (start 117.7 130.7) (end 116.9 129.9) (width 1) (layer "B.Cu") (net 14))
 (segment (start 116.9 115.5) (end 119.8324 112.5676) (width 1) (layer "B.Cu") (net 14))
 (segment (start 116.9 129.9) (end 116.9 115.5) (width 1) (layer "B.Cu") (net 14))
 (segment (start 118.92 133.6) (end 118.92 130.7) (width 1) (layer "B.Cu") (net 14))
 (segment (start 119.8324 112.5676) (end 120.1746 112.5676) (width 1) (layer "B.Cu") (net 14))
 (segment (start 123.7 109.26) (end 124.76 108.2) (width 1) (layer "B.Cu") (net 4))
 (segment (start 123.7 112.82) (end 123.7 109.26) (width 1) (layer "B.Cu") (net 4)))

